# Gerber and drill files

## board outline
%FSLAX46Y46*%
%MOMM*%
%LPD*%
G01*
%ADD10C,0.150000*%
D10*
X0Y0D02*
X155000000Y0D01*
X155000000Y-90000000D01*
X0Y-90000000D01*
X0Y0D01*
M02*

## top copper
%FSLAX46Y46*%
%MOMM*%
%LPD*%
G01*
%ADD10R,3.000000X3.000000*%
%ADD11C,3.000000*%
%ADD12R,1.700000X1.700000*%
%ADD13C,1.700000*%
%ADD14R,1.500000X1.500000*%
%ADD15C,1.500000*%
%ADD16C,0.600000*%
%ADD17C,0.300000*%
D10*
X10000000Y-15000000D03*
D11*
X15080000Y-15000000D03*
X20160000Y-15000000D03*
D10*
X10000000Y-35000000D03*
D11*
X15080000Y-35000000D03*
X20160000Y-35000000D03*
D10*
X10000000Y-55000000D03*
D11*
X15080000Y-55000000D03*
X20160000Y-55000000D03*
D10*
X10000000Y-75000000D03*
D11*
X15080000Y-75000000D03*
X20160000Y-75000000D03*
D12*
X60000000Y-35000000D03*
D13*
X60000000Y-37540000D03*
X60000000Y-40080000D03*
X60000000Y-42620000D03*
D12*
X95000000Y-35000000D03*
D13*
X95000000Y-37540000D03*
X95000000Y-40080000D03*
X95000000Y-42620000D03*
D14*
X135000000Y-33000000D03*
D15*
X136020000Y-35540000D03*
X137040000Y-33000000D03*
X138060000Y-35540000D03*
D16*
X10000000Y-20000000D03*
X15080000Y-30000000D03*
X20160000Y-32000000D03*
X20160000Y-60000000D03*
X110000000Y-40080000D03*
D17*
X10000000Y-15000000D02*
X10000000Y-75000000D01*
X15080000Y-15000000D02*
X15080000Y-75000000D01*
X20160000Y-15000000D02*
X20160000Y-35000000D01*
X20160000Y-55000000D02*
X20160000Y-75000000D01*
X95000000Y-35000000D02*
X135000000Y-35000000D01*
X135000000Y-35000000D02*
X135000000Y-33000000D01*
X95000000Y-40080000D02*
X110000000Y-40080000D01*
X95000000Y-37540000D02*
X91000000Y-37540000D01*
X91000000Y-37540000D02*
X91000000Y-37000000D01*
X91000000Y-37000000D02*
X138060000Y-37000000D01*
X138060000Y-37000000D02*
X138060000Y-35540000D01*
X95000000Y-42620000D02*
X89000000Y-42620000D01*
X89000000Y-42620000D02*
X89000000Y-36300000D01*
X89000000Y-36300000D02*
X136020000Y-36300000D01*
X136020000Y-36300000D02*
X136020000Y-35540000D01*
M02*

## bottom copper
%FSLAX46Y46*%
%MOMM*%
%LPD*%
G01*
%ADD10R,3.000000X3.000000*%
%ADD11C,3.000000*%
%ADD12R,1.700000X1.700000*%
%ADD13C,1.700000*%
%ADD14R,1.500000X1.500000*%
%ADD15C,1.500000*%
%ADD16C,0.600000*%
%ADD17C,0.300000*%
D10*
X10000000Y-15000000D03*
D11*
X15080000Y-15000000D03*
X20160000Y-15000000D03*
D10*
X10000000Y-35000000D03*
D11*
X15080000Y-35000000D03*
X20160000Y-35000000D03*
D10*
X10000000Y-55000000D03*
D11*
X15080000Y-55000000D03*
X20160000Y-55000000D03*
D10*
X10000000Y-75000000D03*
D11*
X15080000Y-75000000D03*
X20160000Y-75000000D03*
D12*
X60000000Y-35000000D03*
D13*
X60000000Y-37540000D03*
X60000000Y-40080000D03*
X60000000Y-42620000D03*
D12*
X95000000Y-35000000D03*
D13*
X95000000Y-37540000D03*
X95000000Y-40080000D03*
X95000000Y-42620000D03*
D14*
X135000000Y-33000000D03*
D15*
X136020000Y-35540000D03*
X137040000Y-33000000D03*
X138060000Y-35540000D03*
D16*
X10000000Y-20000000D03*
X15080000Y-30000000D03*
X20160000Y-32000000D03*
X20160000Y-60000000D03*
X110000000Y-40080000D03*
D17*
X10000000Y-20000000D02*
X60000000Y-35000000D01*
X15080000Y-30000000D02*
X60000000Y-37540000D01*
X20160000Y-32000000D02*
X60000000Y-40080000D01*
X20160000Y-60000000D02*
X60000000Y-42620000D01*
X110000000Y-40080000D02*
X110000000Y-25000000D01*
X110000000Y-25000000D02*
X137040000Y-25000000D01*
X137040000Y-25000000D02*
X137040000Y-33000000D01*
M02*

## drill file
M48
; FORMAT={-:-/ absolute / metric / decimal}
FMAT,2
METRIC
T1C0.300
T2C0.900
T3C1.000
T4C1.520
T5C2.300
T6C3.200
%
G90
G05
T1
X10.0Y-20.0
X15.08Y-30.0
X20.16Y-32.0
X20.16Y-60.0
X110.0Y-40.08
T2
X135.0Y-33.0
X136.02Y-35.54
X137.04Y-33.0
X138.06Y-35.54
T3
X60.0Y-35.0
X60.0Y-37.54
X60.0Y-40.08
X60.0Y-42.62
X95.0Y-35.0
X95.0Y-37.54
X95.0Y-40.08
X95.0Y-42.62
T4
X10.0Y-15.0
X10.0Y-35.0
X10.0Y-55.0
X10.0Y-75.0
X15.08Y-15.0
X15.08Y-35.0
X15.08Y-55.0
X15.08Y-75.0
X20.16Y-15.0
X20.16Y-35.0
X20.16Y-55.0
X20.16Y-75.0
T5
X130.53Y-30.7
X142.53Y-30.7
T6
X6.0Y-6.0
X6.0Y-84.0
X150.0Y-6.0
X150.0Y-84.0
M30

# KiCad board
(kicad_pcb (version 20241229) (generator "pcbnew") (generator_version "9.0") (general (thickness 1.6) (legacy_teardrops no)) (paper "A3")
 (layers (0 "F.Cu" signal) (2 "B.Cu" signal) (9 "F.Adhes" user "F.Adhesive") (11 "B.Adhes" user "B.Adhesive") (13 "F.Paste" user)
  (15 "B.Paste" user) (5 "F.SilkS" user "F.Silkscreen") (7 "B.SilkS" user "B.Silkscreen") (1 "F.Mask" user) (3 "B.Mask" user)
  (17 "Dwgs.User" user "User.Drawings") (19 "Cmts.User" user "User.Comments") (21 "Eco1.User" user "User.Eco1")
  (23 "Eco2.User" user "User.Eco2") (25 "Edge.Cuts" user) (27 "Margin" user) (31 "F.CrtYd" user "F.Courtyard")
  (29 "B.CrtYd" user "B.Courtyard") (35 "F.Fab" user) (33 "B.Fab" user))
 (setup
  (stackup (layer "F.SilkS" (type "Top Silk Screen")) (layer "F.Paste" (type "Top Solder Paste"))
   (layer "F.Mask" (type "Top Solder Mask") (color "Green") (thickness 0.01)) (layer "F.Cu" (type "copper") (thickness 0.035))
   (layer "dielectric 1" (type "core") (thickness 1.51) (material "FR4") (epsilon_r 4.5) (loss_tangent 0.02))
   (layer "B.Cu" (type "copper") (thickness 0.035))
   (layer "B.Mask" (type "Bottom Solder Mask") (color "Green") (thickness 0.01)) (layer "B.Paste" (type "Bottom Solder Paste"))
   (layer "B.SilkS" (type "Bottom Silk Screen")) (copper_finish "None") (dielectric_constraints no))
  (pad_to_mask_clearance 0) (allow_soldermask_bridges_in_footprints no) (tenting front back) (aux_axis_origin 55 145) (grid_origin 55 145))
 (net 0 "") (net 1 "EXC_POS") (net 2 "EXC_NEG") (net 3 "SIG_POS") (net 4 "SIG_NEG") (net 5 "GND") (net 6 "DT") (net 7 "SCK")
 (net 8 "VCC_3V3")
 (gr_rect (start 0 0) (end 155 90) (stroke (width 0.15) (type solid)) (fill no) (layer "Edge.Cuts"))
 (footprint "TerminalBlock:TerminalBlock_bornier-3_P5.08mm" (layer "F.Cu") (at 10 15 0) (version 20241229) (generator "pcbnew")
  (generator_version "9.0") (layer "F.Cu")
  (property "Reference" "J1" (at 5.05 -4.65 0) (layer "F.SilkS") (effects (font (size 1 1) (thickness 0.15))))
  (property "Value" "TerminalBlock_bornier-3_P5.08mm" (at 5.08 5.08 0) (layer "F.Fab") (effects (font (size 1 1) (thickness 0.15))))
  (pad "1" thru_hole rect (at 0 0) (size 3 3) (drill 1.52) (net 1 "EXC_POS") (layers "*.Cu" "*.Mask") (remove_unused_layers no))
  (pad "2" thru_hole circle (at 5.08 0) (size 3 3) (drill 1.52) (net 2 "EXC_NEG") (layers "*.Cu" "*.Mask") (remove_unused_layers no))
  (pad "3" thru_hole circle (at 10.16 0) (size 3 3) (drill 1.52) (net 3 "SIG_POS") (layers "*.Cu" "*.Mask") (remove_unused_layers no)))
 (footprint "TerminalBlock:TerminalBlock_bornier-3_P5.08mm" (layer "F.Cu") (at 10 35 0) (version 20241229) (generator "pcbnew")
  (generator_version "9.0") (layer "F.Cu")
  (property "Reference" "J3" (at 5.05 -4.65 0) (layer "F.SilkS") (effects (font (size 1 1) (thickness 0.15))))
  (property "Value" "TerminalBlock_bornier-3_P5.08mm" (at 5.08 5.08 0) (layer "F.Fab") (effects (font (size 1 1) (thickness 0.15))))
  (pad "1" thru_hole rect (at 0 0) (size 3 3) (drill 1.52) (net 1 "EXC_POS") (layers "*.Cu" "*.Mask") (remove_unused_layers no))
  (pad "2" thru_hole circle (at 5.08 0) (size 3 3) (drill 1.52) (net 2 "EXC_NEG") (layers "*.Cu" "*.Mask") (remove_unused_layers no))
  (pad "3" thru_hole circle (at 10.16 0) (size 3 3) (drill 1.52) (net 3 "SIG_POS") (layers "*.Cu" "*.Mask") (remove_unused_layers no)))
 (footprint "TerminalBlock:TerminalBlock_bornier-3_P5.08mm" (layer "F.Cu") (at 10 55 0) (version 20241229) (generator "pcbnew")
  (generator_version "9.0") (layer "F.Cu")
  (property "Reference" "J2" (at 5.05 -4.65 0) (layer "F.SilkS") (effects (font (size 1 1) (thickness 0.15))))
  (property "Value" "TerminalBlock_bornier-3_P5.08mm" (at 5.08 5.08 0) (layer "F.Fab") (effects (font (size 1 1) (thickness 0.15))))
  (pad "1" thru_hole rect (at 0 0) (size 3 3) (drill 1.52) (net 1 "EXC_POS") (layers "*.Cu" "*.Mask") (remove_unused_layers no))
  (pad "2" thru_hole circle (at 5.08 0) (size 3 3) (drill 1.52) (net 2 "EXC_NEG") (layers "*.Cu" "*.Mask") (remove_unused_layers no))
  (pad "3" thru_hole circle (at 10.16 0) (size 3 3) (drill 1.52) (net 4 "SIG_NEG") (layers "*.Cu" "*.Mask") (remove_unused_layers no)))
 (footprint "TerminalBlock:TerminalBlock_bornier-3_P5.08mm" (layer "F.Cu") (at 10 75 0) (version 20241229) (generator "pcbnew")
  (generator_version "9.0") (layer "F.Cu")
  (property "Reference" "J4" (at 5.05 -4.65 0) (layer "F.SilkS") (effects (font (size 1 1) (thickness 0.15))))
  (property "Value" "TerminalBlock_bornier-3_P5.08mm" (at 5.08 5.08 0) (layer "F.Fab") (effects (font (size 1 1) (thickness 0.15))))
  (pad "1" thru_hole rect (at 0 0) (size 3 3) (drill 1.52) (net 1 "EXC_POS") (layers "*.Cu" "*.Mask") (remove_unused_layers no))
  (pad "2" thru_hole circle (at 5.08 0) (size 3 3) (drill 1.52) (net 2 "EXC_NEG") (layers "*.Cu" "*.Mask") (remove_unused_layers no))
  (pad "3" thru_hole circle (at 10.16 0) (size 3 3) (drill 1.52) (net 4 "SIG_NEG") (layers "*.Cu" "*.Mask") (remove_unused_layers no)))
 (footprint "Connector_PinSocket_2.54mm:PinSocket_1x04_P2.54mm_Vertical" (layer "F.Cu") (at 60 35 0) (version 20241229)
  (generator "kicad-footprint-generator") (layer "F.Cu")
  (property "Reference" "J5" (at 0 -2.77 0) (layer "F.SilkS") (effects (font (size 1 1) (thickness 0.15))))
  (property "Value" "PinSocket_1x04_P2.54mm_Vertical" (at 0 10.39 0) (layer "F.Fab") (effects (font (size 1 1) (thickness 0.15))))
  (pad "1" thru_hole rect (at 0 0) (size 1.7 1.7) (drill 1) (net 1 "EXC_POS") (layers "*.Cu" "*.Mask") (remove_unused_layers no))
  (pad "2" thru_hole circle (at 0 2.54) (size 1.7 1.7) (drill 1) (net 2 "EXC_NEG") (layers "*.Cu" "*.Mask") (remove_unused_layers no))
  (pad "3" thru_hole circle (at 0 5.08) (size 1.7 1.7) (drill 1) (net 3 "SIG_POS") (layers "*.Cu" "*.Mask") (remove_unused_layers no))
  (pad "4" thru_hole circle (at 0 7.62) (size 1.7 1.7) (drill 1) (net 4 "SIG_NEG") (layers "*.Cu" "*.Mask") (remove_unused_layers no)))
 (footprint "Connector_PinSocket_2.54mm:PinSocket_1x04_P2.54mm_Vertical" (layer "F.Cu") (at 95 35 0) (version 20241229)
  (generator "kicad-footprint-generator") (layer "F.Cu")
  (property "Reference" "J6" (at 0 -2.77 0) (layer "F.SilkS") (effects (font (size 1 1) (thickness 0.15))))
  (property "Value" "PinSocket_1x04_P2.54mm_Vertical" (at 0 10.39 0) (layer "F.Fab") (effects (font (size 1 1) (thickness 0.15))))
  (pad "1" thru_hole rect (at 0 0) (size 1.7 1.7) (drill 1) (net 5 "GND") (layers "*.Cu" "*.Mask") (remove_unused_layers no))
  (pad "2" thru_hole circle (at 0 2.54) (size 1.7 1.7) (drill 1) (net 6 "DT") (layers "*.Cu" "*.Mask") (remove_unused_layers no))
  (pad "3" thru_hole circle (at 0 5.08) (size 1.7 1.7) (drill 1) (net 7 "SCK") (layers "*.Cu" "*.Mask") (remove_unused_layers no))
  (pad "4" thru_hole circle (at 0 7.62) (size 1.7 1.7) (drill 1) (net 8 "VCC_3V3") (layers "*.Cu" "*.Mask") (remove_unused_layers no)))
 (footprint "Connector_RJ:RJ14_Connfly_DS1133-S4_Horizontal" (layer "F.Cu") (at 135 33 0) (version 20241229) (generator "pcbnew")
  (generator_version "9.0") (layer "F.Cu")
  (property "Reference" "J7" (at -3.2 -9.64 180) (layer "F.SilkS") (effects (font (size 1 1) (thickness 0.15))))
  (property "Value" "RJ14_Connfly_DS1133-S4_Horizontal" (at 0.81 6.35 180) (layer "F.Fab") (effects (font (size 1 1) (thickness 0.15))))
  (pad "" np_thru_hole circle (at -4.47 -2.3 180) (size 2.3 2.3) (drill 2.3) (layers "*.Cu" "*.Mask"))
  (pad "" np_thru_hole circle (at 7.53 -2.3 180) (size 2.3 2.3) (drill 2.3) (layers "*.Cu" "*.Mask"))
  (pad "1" thru_hole rect (at 0 0 180) (size 1.5 1.5) (drill 0.9) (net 5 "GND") (layers "*.Cu" "*.Mask") (remove_unused_layers no))
  (pad "2" thru_hole circle (at 1.02 2.54 180) (size 1.5 1.5) (drill 0.9) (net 8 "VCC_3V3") (layers "*.Cu" "*.Mask")
   (remove_unused_layers no))
  (pad "3" thru_hole circle (at 2.04 0 180) (size 1.5 1.5) (drill 0.9) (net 7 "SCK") (layers "*.Cu" "*.Mask") (remove_unused_layers no))
  (pad "4" thru_hole circle (at 3.06 2.54 180) (size 1.5 1.5) (drill 0.9) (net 6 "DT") (layers "*.Cu" "*.Mask") (remove_unused_layers no)))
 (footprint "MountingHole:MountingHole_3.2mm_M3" (layer "F.Cu") (at 6 6 0) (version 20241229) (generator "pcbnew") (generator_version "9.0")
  (layer "F.Cu")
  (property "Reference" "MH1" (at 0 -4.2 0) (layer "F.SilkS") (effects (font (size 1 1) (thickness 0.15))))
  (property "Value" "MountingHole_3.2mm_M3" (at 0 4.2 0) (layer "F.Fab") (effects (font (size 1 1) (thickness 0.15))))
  (pad "" np_thru_hole circle (at 0 0) (size 3.2 3.2) (drill 3.2) (layers "*.Cu" "*.Mask")))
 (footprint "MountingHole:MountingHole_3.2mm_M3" (layer "F.Cu") (at 150 6 0) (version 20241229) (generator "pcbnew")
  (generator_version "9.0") (layer "F.Cu")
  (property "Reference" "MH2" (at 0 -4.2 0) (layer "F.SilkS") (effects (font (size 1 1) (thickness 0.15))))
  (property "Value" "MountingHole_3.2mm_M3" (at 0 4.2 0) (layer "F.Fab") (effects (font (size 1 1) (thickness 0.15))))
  (pad "" np_thru_hole circle (at 0 0) (size 3.2 3.2) (drill 3.2) (layers "*.Cu" "*.Mask")))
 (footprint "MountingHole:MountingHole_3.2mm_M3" (layer "F.Cu") (at 6 84 0) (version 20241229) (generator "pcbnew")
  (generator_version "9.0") (layer "F.Cu")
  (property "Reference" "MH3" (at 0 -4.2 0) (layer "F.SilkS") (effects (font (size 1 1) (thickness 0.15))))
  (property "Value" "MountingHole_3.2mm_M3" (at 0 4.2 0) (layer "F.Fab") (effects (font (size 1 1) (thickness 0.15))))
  (pad "" np_thru_hole circle (at 0 0) (size 3.2 3.2) (drill 3.2) (layers "*.Cu" "*.Mask")))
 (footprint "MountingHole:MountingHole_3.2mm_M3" (layer "F.Cu") (at 150 84 0) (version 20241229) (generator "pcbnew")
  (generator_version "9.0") (layer "F.Cu")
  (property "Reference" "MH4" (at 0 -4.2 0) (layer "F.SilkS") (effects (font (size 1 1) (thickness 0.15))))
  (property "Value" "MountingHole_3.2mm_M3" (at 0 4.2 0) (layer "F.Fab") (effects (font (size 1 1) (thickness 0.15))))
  (pad "" np_thru_hole circle (at 0 0) (size 3.2 3.2) (drill 3.2) (layers "*.Cu" "*.Mask")))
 (segment (start 10 15) (end 10 75) (width 0.3) (layer "F.Cu") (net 1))
 (segment (start 10 20) (end 60 35) (width 0.3) (layer "B.Cu") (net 1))
 (segment (start 15.08 15) (end 15.08 75) (width 0.3) (layer "F.Cu") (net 2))
 (segment (start 15.08 30) (end 60 37.54) (width 0.3) (layer "B.Cu") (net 2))
 (segment (start 20.16 15) (end 20.16 35) (width 0.3) (layer "F.Cu") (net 3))
 (segment (start 20.16 32) (end 60 40.08) (width 0.3) (layer "B.Cu") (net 3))
 (segment (start 20.16 55) (end 20.16 75) (width 0.3) (layer "F.Cu") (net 4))
 (segment (start 20.16 60) (end 60 42.62) (width 0.3) (layer "B.Cu") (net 4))
 (segment (start 95 35) (end 135 35) (width 0.3) (layer "F.Cu") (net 5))
 (segment (start 135 35) (end 135 33) (width 0.3) (layer "F.Cu") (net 5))
 (segment (start 95 40.08) (end 110 40.08) (width 0.3) (layer "F.Cu") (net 7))
 (segment (start 110 40.08) (end 110 25) (width 0.3) (layer "B.Cu") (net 7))
 (segment (start 110 25) (end 137.04 25) (width 0.3) (layer "B.Cu") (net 7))
 (segment (start 137.04 25) (end 137.04 33) (width 0.3) (layer "B.Cu") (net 7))
 (segment (start 95 37.54) (end 91 37.54) (width 0.3) (layer "F.Cu") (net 6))
 (segment (start 91 37.54) (end 91 37) (width 0.3) (layer "F.Cu") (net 6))
 (segment (start 91 37) (end 138.06 37) (width 0.3) (layer "F.Cu") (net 6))
 (segment (start 138.06 37) (end 138.06 35.54) (width 0.3) (layer "F.Cu") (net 6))
 (segment (start 95 42.62) (end 89 42.62) (width 0.3) (layer "F.Cu") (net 8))
 (segment (start 89 42.62) (end 89 36.3) (width 0.3) (layer "F.Cu") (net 8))
 (segment (start 89 36.3) (end 136.02 36.3) (width 0.3) (layer "F.Cu") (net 8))
 (segment (start 136.02 36.3) (end 136.02 35.54) (width 0.3) (layer "F.Cu") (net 8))
 (via (at 10 20) (size 0.6) (drill 0.3) (layers "F.Cu" "B.Cu") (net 1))
 (via (at 15.08 30) (size 0.6) (drill 0.3) (layers "F.Cu" "B.Cu") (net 2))
 (via (at 20.16 32) (size 0.6) (drill 0.3) (layers "F.Cu" "B.Cu") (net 3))
 (via (at 20.16 60) (size 0.6) (drill 0.3) (layers "F.Cu" "B.Cu") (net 4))
 (via (at 110 40.08) (size 0.6) (drill 0.3) (layers "F.Cu" "B.Cu") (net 7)))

